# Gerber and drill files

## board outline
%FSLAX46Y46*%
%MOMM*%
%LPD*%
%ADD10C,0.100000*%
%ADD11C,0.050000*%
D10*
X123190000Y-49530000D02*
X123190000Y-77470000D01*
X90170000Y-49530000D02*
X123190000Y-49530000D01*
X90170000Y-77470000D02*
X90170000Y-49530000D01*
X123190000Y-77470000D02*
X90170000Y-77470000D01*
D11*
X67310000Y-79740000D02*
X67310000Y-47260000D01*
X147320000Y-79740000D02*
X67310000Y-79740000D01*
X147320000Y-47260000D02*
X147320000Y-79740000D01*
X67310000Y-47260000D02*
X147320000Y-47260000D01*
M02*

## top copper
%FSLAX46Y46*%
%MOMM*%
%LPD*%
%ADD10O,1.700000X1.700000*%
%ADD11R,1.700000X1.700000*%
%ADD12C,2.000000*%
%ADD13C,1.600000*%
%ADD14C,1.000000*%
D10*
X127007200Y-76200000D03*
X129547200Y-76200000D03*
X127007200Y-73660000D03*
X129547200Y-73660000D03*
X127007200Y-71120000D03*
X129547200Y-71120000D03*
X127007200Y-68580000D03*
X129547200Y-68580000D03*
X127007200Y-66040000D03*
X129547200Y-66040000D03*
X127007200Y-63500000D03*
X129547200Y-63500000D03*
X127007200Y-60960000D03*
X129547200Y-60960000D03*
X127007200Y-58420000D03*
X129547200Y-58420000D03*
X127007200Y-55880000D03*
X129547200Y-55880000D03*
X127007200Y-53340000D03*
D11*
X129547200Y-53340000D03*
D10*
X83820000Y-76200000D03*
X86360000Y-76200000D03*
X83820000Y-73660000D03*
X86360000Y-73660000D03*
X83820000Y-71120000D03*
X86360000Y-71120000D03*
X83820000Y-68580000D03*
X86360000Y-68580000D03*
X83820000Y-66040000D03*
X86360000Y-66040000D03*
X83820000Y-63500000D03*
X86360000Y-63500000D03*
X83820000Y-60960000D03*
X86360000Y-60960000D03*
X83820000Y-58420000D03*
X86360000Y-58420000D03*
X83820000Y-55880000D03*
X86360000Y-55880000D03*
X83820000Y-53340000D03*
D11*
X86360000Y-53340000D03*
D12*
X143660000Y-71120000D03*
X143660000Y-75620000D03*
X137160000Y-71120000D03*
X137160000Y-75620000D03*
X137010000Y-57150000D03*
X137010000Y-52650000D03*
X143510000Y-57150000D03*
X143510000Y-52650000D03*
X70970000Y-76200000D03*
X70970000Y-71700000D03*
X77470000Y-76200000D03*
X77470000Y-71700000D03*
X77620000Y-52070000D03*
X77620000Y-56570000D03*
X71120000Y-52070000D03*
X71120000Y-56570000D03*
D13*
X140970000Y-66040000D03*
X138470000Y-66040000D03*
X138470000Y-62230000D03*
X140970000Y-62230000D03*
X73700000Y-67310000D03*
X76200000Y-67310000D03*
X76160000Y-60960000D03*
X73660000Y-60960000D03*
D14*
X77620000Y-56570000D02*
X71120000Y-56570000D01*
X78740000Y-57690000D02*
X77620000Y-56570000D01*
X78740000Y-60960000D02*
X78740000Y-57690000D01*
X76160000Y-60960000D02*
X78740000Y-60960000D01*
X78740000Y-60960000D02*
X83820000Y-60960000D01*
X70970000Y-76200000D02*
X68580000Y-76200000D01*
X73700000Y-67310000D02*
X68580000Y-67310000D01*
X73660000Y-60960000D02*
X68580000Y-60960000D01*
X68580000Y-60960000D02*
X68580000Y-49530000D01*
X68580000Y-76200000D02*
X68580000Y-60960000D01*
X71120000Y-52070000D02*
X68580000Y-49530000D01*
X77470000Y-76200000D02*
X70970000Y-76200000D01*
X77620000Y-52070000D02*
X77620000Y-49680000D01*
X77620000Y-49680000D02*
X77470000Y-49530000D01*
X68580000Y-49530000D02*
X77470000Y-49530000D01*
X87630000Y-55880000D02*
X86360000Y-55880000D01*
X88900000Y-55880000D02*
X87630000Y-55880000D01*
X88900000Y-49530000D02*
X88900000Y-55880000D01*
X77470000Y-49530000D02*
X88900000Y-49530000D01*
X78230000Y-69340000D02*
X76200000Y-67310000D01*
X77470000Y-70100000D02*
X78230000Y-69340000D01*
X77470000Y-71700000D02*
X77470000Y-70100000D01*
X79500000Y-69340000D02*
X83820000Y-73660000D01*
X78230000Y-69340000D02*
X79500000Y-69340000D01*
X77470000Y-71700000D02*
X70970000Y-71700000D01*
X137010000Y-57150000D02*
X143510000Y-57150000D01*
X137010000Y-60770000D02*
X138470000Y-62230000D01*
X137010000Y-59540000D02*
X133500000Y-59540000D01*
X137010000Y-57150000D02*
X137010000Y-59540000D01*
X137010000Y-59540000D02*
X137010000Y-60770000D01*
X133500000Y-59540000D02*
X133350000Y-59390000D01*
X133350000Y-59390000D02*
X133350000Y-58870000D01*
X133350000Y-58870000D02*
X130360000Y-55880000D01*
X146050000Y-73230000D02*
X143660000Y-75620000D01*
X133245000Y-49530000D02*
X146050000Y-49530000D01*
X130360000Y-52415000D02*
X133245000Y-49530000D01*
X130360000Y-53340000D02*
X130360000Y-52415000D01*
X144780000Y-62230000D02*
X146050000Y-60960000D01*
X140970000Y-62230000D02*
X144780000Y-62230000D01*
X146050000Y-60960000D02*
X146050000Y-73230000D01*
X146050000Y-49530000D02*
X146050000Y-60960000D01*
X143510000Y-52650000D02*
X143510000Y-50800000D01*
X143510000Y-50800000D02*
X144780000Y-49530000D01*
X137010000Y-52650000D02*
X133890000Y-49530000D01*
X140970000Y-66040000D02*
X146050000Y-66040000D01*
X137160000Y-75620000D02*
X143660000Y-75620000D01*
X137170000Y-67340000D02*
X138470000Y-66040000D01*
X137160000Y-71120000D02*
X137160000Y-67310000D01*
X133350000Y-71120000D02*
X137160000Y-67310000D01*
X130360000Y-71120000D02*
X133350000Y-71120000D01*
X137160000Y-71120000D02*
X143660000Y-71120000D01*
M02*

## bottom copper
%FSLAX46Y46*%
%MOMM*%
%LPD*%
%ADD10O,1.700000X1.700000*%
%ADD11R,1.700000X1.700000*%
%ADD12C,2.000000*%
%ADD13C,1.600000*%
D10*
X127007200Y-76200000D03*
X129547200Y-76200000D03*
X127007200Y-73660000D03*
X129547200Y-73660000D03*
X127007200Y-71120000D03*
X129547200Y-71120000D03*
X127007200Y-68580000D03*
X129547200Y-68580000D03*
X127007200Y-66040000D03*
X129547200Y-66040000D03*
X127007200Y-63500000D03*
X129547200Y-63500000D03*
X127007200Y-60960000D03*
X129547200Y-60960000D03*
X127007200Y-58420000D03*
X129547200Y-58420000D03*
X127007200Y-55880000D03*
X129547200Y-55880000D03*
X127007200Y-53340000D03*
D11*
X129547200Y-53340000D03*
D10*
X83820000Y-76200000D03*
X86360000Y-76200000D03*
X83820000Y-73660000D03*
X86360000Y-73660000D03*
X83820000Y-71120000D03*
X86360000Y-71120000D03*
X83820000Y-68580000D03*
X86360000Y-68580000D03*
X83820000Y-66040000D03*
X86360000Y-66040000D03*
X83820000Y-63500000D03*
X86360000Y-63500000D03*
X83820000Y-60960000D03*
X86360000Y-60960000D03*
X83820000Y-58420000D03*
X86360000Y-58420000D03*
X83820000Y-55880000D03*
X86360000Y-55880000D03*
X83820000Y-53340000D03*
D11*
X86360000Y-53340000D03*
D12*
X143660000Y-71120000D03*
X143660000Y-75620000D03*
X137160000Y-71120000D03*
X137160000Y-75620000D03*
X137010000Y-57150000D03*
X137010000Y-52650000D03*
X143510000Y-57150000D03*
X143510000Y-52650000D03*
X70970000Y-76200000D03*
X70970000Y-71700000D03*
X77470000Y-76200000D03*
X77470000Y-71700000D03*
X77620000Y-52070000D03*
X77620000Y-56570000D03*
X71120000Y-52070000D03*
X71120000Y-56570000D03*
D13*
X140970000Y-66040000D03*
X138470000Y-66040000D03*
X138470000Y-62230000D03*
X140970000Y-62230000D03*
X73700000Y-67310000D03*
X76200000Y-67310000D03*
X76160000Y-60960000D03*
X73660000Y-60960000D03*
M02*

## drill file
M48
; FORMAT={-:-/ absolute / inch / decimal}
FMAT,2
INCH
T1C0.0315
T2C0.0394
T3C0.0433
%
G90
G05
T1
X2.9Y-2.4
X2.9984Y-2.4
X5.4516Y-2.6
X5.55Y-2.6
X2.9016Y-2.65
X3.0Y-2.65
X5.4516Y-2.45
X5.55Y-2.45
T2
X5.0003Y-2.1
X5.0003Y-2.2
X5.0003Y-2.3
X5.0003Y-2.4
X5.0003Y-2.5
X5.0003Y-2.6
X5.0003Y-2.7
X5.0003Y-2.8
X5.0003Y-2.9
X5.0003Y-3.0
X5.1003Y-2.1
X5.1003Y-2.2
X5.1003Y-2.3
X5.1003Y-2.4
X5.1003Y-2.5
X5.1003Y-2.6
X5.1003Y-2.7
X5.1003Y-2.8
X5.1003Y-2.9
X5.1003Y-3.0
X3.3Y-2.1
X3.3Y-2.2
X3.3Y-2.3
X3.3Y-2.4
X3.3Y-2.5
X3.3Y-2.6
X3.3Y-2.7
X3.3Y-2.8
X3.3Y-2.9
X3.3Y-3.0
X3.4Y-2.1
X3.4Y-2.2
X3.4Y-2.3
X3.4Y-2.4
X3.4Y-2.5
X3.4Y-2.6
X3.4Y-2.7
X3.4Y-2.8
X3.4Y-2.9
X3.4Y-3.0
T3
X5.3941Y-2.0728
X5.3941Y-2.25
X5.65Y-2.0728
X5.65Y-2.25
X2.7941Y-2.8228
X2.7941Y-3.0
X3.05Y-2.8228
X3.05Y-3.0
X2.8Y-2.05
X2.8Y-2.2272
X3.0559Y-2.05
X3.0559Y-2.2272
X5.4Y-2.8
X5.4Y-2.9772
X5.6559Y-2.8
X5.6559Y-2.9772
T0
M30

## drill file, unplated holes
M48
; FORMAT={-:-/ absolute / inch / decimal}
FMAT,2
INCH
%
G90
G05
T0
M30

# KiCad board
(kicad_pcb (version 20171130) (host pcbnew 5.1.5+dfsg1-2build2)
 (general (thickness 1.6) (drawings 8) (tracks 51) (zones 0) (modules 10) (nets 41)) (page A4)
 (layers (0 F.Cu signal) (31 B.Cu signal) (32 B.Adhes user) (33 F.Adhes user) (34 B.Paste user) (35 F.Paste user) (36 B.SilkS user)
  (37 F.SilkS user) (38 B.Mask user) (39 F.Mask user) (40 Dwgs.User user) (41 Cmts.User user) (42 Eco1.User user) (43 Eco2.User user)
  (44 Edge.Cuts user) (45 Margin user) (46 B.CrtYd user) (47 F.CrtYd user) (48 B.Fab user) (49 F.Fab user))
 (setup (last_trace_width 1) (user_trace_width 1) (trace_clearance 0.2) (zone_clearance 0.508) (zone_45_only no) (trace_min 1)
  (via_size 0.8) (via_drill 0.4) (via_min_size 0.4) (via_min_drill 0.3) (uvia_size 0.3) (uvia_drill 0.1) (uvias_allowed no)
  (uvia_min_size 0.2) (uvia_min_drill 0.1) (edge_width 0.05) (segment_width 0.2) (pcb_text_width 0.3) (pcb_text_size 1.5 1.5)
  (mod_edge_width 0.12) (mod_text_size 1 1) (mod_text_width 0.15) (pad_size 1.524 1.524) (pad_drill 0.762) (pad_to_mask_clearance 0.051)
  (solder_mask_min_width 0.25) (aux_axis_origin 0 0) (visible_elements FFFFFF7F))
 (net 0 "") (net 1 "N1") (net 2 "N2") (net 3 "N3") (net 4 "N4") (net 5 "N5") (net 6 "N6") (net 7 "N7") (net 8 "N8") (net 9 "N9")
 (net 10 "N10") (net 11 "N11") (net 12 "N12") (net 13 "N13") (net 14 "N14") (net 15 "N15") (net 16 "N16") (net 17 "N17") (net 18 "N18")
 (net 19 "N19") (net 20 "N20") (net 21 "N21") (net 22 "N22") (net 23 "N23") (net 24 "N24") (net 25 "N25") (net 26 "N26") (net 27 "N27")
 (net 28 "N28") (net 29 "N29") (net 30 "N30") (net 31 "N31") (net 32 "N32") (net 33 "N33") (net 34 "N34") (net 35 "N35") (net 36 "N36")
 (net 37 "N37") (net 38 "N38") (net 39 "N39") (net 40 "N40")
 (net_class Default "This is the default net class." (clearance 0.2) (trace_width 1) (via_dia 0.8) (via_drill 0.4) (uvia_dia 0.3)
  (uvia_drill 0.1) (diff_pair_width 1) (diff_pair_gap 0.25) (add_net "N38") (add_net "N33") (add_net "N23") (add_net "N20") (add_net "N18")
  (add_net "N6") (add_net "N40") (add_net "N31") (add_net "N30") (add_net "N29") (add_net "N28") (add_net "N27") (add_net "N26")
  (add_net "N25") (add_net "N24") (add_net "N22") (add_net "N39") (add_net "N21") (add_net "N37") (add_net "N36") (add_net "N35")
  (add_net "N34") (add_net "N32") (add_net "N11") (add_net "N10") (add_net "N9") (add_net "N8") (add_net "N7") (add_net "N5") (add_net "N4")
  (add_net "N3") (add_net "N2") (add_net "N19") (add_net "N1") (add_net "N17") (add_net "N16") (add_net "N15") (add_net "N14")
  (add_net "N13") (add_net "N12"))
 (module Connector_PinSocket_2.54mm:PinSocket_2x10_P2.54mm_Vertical (layer F.Cu) (at 129.5472 53.34)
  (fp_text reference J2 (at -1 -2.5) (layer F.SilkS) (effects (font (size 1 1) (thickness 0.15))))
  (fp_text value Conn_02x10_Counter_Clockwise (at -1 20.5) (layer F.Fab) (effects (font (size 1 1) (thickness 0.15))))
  (pad 20 thru_hole oval (at -2.54 22.86) (size 1.7 1.7) (drill 1) (layers *.Cu *.Mask) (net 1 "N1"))
  (pad 19 thru_hole oval (at 0 22.86) (size 1.7 1.7) (drill 1) (layers *.Cu *.Mask) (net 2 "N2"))
  (pad 18 thru_hole oval (at -2.54 20.32) (size 1.7 1.7) (drill 1) (layers *.Cu *.Mask) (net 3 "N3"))
  (pad 17 thru_hole oval (at 0 20.32) (size 1.7 1.7) (drill 1) (layers *.Cu *.Mask) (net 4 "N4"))
  (pad 16 thru_hole oval (at -2.54 17.78) (size 1.7 1.7) (drill 1) (layers *.Cu *.Mask) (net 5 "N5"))
  (pad 15 thru_hole oval (at 0 17.78) (size 1.7 1.7) (drill 1) (layers *.Cu *.Mask) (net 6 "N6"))
  (pad 14 thru_hole oval (at -2.54 15.24) (size 1.7 1.7) (drill 1) (layers *.Cu *.Mask) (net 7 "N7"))
  (pad 13 thru_hole oval (at 0 15.24) (size 1.7 1.7) (drill 1) (layers *.Cu *.Mask) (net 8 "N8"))
  (pad 12 thru_hole oval (at -2.54 12.7) (size 1.7 1.7) (drill 1) (layers *.Cu *.Mask) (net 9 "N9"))
  (pad 11 thru_hole oval (at 0 12.7) (size 1.7 1.7) (drill 1) (layers *.Cu *.Mask) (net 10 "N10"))
  (pad 10 thru_hole oval (at -2.54 10.16) (size 1.7 1.7) (drill 1) (layers *.Cu *.Mask) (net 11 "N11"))
  (pad 9 thru_hole oval (at 0 10.16) (size 1.7 1.7) (drill 1) (layers *.Cu *.Mask) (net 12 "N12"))
  (pad 8 thru_hole oval (at -2.54 7.62) (size 1.7 1.7) (drill 1) (layers *.Cu *.Mask) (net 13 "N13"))
  (pad 7 thru_hole oval (at 0 7.62) (size 1.7 1.7) (drill 1) (layers *.Cu *.Mask) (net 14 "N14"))
  (pad 6 thru_hole oval (at -2.54 5.08) (size 1.7 1.7) (drill 1) (layers *.Cu *.Mask) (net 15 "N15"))
  (pad 5 thru_hole oval (at 0 5.08) (size 1.7 1.7) (drill 1) (layers *.Cu *.Mask) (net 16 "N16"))
  (pad 4 thru_hole oval (at -2.54 2.54) (size 1.7 1.7) (drill 1) (layers *.Cu *.Mask) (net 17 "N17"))
  (pad 3 thru_hole oval (at 0 2.54) (size 1.7 1.7) (drill 1) (layers *.Cu *.Mask) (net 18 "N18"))
  (pad 2 thru_hole oval (at -2.54 0) (size 1.7 1.7) (drill 1) (layers *.Cu *.Mask) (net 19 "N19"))
  (pad 1 thru_hole rect (at 0 0) (size 1.7 1.7) (drill 1) (layers *.Cu *.Mask) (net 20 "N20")))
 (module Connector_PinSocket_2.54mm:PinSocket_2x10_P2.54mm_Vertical (layer F.Cu) (at 86.36 53.34)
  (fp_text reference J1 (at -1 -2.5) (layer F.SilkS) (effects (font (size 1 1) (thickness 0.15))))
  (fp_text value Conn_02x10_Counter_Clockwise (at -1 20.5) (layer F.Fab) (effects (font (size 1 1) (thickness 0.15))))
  (pad 20 thru_hole oval (at -2.54 22.86) (size 1.7 1.7) (drill 1) (layers *.Cu *.Mask) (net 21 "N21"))
  (pad 19 thru_hole oval (at 0 22.86) (size 1.7 1.7) (drill 1) (layers *.Cu *.Mask) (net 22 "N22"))
  (pad 18 thru_hole oval (at -2.54 20.32) (size 1.7 1.7) (drill 1) (layers *.Cu *.Mask) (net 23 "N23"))
  (pad 17 thru_hole oval (at 0 20.32) (size 1.7 1.7) (drill 1) (layers *.Cu *.Mask) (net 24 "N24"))
  (pad 16 thru_hole oval (at -2.54 17.78) (size 1.7 1.7) (drill 1) (layers *.Cu *.Mask) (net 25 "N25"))
  (pad 15 thru_hole oval (at 0 17.78) (size 1.7 1.7) (drill 1) (layers *.Cu *.Mask) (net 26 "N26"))
  (pad 14 thru_hole oval (at -2.54 15.24) (size 1.7 1.7) (drill 1) (layers *.Cu *.Mask) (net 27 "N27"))
  (pad 13 thru_hole oval (at 0 15.24) (size 1.7 1.7) (drill 1) (layers *.Cu *.Mask) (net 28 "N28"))
  (pad 12 thru_hole oval (at -2.54 12.7) (size 1.7 1.7) (drill 1) (layers *.Cu *.Mask) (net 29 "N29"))
  (pad 11 thru_hole oval (at 0 12.7) (size 1.7 1.7) (drill 1) (layers *.Cu *.Mask) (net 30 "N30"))
  (pad 10 thru_hole oval (at -2.54 10.16) (size 1.7 1.7) (drill 1) (layers *.Cu *.Mask) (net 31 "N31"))
  (pad 9 thru_hole oval (at 0 10.16) (size 1.7 1.7) (drill 1) (layers *.Cu *.Mask) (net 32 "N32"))
  (pad 8 thru_hole oval (at -2.54 7.62) (size 1.7 1.7) (drill 1) (layers *.Cu *.Mask) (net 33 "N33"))
  (pad 7 thru_hole oval (at 0 7.62) (size 1.7 1.7) (drill 1) (layers *.Cu *.Mask) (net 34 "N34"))
  (pad 6 thru_hole oval (at -2.54 5.08) (size 1.7 1.7) (drill 1) (layers *.Cu *.Mask) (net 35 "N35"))
  (pad 5 thru_hole oval (at 0 5.08) (size 1.7 1.7) (drill 1) (layers *.Cu *.Mask) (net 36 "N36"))
  (pad 4 thru_hole oval (at -2.54 2.54) (size 1.7 1.7) (drill 1) (layers *.Cu *.Mask) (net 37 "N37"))
  (pad 3 thru_hole oval (at 0 2.54) (size 1.7 1.7) (drill 1) (layers *.Cu *.Mask) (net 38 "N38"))
  (pad 2 thru_hole oval (at -2.54 0) (size 1.7 1.7) (drill 1) (layers *.Cu *.Mask) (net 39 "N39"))
  (pad 1 thru_hole rect (at 0 0) (size 1.7 1.7) (drill 1) (layers *.Cu *.Mask) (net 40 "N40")))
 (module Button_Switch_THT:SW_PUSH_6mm (layer F.Cu) (at 137.16 71.12)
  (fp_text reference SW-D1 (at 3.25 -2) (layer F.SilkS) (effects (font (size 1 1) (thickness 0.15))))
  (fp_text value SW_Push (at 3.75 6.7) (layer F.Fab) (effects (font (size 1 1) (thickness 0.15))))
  (pad 1 thru_hole circle (at 6.5 0 90) (size 2 2) (drill 1.1) (layers *.Cu *.Mask) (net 6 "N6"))
  (pad 2 thru_hole circle (at 6.5 4.5 90) (size 2 2) (drill 1.1) (layers *.Cu *.Mask) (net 20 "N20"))
  (pad 1 thru_hole circle (at 0 0 90) (size 2 2) (drill 1.1) (layers *.Cu *.Mask) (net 6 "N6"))
  (pad 2 thru_hole circle (at 0 4.5 90) (size 2 2) (drill 1.1) (layers *.Cu *.Mask) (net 20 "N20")))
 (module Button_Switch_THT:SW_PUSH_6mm (layer F.Cu) (at 143.51 57.15 180)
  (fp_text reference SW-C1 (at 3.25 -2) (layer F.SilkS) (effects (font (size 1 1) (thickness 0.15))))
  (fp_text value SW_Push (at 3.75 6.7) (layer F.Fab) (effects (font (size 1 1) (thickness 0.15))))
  (pad 1 thru_hole circle (at 6.5 0 270) (size 2 2) (drill 1.1) (layers *.Cu *.Mask) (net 18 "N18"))
  (pad 2 thru_hole circle (at 6.5 4.5 270) (size 2 2) (drill 1.1) (layers *.Cu *.Mask) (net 20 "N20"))
  (pad 1 thru_hole circle (at 0 0 270) (size 2 2) (drill 1.1) (layers *.Cu *.Mask) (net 18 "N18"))
  (pad 2 thru_hole circle (at 0 4.5 270) (size 2 2) (drill 1.1) (layers *.Cu *.Mask) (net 20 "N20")))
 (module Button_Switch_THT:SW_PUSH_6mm (layer F.Cu) (at 77.47 76.2 180)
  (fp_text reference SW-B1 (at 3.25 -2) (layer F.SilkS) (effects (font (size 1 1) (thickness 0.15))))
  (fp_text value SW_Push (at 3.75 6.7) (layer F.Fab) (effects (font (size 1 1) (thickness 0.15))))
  (pad 1 thru_hole circle (at 6.5 0 270) (size 2 2) (drill 1.1) (layers *.Cu *.Mask) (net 38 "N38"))
  (pad 2 thru_hole circle (at 6.5 4.5 270) (size 2 2) (drill 1.1) (layers *.Cu *.Mask) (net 23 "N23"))
  (pad 1 thru_hole circle (at 0 0 270) (size 2 2) (drill 1.1) (layers *.Cu *.Mask) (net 38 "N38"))
  (pad 2 thru_hole circle (at 0 4.5 270) (size 2 2) (drill 1.1) (layers *.Cu *.Mask) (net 23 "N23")))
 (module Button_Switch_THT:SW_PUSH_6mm (layer F.Cu) (at 71.12 52.07)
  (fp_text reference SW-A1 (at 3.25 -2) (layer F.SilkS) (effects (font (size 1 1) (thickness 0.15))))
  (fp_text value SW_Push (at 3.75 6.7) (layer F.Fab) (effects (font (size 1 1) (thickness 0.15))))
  (pad 1 thru_hole circle (at 6.5 0 90) (size 2 2) (drill 1.1) (layers *.Cu *.Mask) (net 38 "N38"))
  (pad 2 thru_hole circle (at 6.5 4.5 90) (size 2 2) (drill 1.1) (layers *.Cu *.Mask) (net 33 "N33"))
  (pad 1 thru_hole circle (at 0 0 90) (size 2 2) (drill 1.1) (layers *.Cu *.Mask) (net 38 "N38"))
  (pad 2 thru_hole circle (at 0 4.5 90) (size 2 2) (drill 1.1) (layers *.Cu *.Mask) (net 33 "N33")))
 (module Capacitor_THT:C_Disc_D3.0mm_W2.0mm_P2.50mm (layer F.Cu) (at 138.47 66.04)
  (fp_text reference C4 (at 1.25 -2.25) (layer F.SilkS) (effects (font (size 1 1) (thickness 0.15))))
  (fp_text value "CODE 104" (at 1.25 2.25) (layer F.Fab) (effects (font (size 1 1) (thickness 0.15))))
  (pad 2 thru_hole circle (at 2.5 0) (size 1.6 1.6) (drill 0.8) (layers *.Cu *.Mask) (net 20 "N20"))
  (pad 1 thru_hole circle (at 0 0) (size 1.6 1.6) (drill 0.8) (layers *.Cu *.Mask) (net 6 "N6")))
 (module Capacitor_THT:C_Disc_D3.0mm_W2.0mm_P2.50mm (layer F.Cu) (at 140.97 62.23 180)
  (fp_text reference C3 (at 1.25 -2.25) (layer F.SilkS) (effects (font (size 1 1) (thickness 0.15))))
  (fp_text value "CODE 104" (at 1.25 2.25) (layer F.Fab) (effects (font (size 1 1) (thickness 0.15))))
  (pad 2 thru_hole circle (at 2.5 0 180) (size 1.6 1.6) (drill 0.8) (layers *.Cu *.Mask) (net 18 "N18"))
  (pad 1 thru_hole circle (at 0 0 180) (size 1.6 1.6) (drill 0.8) (layers *.Cu *.Mask) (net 20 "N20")))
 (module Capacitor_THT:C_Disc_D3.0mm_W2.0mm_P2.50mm (layer F.Cu) (at 76.2 67.31 180)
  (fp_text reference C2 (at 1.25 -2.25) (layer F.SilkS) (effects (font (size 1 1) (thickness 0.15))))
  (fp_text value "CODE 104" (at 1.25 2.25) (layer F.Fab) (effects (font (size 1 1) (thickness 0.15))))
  (pad 2 thru_hole circle (at 2.5 0 180) (size 1.6 1.6) (drill 0.8) (layers *.Cu *.Mask) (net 38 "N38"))
  (pad 1 thru_hole circle (at 0 0 180) (size 1.6 1.6) (drill 0.8) (layers *.Cu *.Mask) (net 23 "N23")))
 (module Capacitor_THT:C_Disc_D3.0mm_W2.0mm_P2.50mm (layer F.Cu) (at 73.66 60.96)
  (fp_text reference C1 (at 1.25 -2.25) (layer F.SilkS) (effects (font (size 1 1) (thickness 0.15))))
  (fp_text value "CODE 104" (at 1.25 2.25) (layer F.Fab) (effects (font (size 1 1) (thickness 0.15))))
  (pad 2 thru_hole circle (at 2.5 0) (size 1.6 1.6) (drill 0.8) (layers *.Cu *.Mask) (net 33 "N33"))
  (pad 1 thru_hole circle (at 0 0) (size 1.6 1.6) (drill 0.8) (layers *.Cu *.Mask) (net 38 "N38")))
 (gr_line (start 123.19 49.53) (end 123.19 77.47) (layer Edge.Cuts) (width 0.1))
 (gr_line (start 90.17 49.53) (end 123.19 49.53) (layer Edge.Cuts) (width 0.1))
 (gr_line (start 90.17 77.47) (end 90.17 49.53) (layer Edge.Cuts) (width 0.1))
 (gr_line (start 123.19 77.47) (end 90.17 77.47) (layer Edge.Cuts) (width 0.1))
 (gr_line (start 67.31 79.74) (end 67.31 47.26) (layer Edge.Cuts) (width 0.05))
 (gr_line (start 147.32 79.74) (end 67.31 79.74) (layer Edge.Cuts) (width 0.05))
 (gr_line (start 147.32 47.26) (end 147.32 79.74) (layer Edge.Cuts) (width 0.05))
 (gr_line (start 67.31 47.26) (end 147.32 47.26) (layer Edge.Cuts) (width 0.05))
 (segment (start 77.62 56.57) (end 71.12 56.57) (width 1) (layer F.Cu) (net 33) (status 30))
 (segment (start 78.74 57.69) (end 77.62 56.57) (width 1) (layer F.Cu) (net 33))
 (segment (start 78.74 60.96) (end 78.74 57.69) (width 1) (layer F.Cu) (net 33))
 (segment (start 76.16 60.96) (end 78.74 60.96) (width 1) (layer F.Cu) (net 33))
 (segment (start 78.74 60.96) (end 83.82 60.96) (width 1) (layer F.Cu) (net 33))
 (segment (start 70.97 76.2) (end 68.58 76.2) (width 1) (layer F.Cu) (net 38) (status 10))
 (segment (start 73.7 67.31) (end 68.58 67.31) (width 1) (layer F.Cu) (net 38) (status 10))
 (segment (start 73.66 60.96) (end 68.58 60.96) (width 1) (layer F.Cu) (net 38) (status 10))
 (segment (start 68.58 60.96) (end 68.58 49.53) (width 1) (layer F.Cu) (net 38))
 (segment (start 68.58 76.2) (end 68.58 60.96) (width 1) (layer F.Cu) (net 38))
 (segment (start 71.12 52.07) (end 68.58 49.53) (width 1) (layer F.Cu) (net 38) (status 10))
 (segment (start 77.47 76.2) (end 70.97 76.2) (width 1) (layer F.Cu) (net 38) (status 30))
 (segment (start 77.62 52.07) (end 77.62 49.68) (width 1) (layer F.Cu) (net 38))
 (segment (start 77.62 49.68) (end 77.47 49.53) (width 1) (layer F.Cu) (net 38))
 (segment (start 68.58 49.53) (end 77.47 49.53) (width 1) (layer F.Cu) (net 38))
 (segment (start 87.63 55.88) (end 86.36 55.88) (width 1) (layer F.Cu) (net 38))
 (segment (start 88.9 55.88) (end 87.63 55.88) (width 1) (layer F.Cu) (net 38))
 (segment (start 88.9 49.53) (end 88.9 55.88) (width 1) (layer F.Cu) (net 38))
 (segment (start 77.47 49.53) (end 88.9 49.53) (width 1) (layer F.Cu) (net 38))
 (segment (start 78.23 69.34) (end 76.2 67.31) (width 1) (layer F.Cu) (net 23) (status 20))
 (segment (start 77.47 70.1) (end 78.23 69.34) (width 1) (layer F.Cu) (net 23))
 (segment (start 77.47 71.7) (end 77.47 70.1) (width 1) (layer F.Cu) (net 23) (status 10))
 (segment (start 79.5 69.34) (end 83.82 73.66) (width 1) (layer F.Cu) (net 23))
 (segment (start 78.23 69.34) (end 79.5 69.34) (width 1) (layer F.Cu) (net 23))
 (segment (start 77.47 71.7) (end 70.97 71.7) (width 1) (layer F.Cu) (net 23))
 (segment (start 137.01 57.15) (end 143.51 57.15) (width 1) (layer F.Cu) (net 18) (status 30))
 (segment (start 137.01 60.77) (end 138.47 62.23) (width 1) (layer F.Cu) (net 18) (status 20))
 (segment (start 137.01 59.54) (end 133.5 59.54) (width 1) (layer F.Cu) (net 18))
 (segment (start 137.01 57.15) (end 137.01 59.54) (width 1) (layer F.Cu) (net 18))
 (segment (start 137.01 59.54) (end 137.01 60.77) (width 1) (layer F.Cu) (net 18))
 (segment (start 133.5 59.54) (end 133.35 59.39) (width 1) (layer F.Cu) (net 18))
 (segment (start 133.35 59.39) (end 133.35 58.87) (width 1) (layer F.Cu) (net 18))
 (segment (start 133.35 58.87) (end 130.36 55.88) (width 1) (layer F.Cu) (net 18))
 (segment (start 146.05 73.23) (end 143.66 75.62) (width 1) (layer F.Cu) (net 20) (status 20))
 (segment (start 133.245 49.53) (end 146.05 49.53) (width 1) (layer F.Cu) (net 20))
 (segment (start 130.36 52.415) (end 133.245 49.53) (width 1) (layer F.Cu) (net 20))
 (segment (start 130.36 53.34) (end 130.36 52.415) (width 1) (layer F.Cu) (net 20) (status 10))
 (segment (start 144.78 62.23) (end 146.05 60.96) (width 1) (layer F.Cu) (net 20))
 (segment (start 140.97 62.23) (end 144.78 62.23) (width 1) (layer F.Cu) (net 20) (status 10))
 (segment (start 146.05 60.96) (end 146.05 73.23) (width 1) (layer F.Cu) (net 20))
 (segment (start 146.05 49.53) (end 146.05 60.96) (width 1) (layer F.Cu) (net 20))
 (segment (start 143.51 52.65) (end 143.51 50.8) (width 1) (layer F.Cu) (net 20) (status 10))
 (segment (start 143.51 50.8) (end 144.78 49.53) (width 1) (layer F.Cu) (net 20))
 (segment (start 137.01 52.65) (end 133.89 49.53) (width 1) (layer F.Cu) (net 20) (status 10))
 (segment (start 140.97 66.04) (end 146.05 66.04) (width 1) (layer F.Cu) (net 20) (status 10))
 (segment (start 137.16 75.62) (end 143.66 75.62) (width 1) (layer F.Cu) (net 20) (status 30))
 (segment (start 137.17 67.34) (end 138.47 66.04) (width 1) (layer F.Cu) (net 6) (status 20))
 (segment (start 137.16 71.12) (end 137.16 67.31) (width 1) (layer F.Cu) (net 6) (status 10))
 (segment (start 133.35 71.12) (end 137.16 67.31) (width 1) (layer F.Cu) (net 6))
 (segment (start 130.36 71.12) (end 133.35 71.12) (width 1) (layer F.Cu) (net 6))
 (segment (start 137.16 71.12) (end 143.66 71.12) (width 1) (layer F.Cu) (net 6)))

